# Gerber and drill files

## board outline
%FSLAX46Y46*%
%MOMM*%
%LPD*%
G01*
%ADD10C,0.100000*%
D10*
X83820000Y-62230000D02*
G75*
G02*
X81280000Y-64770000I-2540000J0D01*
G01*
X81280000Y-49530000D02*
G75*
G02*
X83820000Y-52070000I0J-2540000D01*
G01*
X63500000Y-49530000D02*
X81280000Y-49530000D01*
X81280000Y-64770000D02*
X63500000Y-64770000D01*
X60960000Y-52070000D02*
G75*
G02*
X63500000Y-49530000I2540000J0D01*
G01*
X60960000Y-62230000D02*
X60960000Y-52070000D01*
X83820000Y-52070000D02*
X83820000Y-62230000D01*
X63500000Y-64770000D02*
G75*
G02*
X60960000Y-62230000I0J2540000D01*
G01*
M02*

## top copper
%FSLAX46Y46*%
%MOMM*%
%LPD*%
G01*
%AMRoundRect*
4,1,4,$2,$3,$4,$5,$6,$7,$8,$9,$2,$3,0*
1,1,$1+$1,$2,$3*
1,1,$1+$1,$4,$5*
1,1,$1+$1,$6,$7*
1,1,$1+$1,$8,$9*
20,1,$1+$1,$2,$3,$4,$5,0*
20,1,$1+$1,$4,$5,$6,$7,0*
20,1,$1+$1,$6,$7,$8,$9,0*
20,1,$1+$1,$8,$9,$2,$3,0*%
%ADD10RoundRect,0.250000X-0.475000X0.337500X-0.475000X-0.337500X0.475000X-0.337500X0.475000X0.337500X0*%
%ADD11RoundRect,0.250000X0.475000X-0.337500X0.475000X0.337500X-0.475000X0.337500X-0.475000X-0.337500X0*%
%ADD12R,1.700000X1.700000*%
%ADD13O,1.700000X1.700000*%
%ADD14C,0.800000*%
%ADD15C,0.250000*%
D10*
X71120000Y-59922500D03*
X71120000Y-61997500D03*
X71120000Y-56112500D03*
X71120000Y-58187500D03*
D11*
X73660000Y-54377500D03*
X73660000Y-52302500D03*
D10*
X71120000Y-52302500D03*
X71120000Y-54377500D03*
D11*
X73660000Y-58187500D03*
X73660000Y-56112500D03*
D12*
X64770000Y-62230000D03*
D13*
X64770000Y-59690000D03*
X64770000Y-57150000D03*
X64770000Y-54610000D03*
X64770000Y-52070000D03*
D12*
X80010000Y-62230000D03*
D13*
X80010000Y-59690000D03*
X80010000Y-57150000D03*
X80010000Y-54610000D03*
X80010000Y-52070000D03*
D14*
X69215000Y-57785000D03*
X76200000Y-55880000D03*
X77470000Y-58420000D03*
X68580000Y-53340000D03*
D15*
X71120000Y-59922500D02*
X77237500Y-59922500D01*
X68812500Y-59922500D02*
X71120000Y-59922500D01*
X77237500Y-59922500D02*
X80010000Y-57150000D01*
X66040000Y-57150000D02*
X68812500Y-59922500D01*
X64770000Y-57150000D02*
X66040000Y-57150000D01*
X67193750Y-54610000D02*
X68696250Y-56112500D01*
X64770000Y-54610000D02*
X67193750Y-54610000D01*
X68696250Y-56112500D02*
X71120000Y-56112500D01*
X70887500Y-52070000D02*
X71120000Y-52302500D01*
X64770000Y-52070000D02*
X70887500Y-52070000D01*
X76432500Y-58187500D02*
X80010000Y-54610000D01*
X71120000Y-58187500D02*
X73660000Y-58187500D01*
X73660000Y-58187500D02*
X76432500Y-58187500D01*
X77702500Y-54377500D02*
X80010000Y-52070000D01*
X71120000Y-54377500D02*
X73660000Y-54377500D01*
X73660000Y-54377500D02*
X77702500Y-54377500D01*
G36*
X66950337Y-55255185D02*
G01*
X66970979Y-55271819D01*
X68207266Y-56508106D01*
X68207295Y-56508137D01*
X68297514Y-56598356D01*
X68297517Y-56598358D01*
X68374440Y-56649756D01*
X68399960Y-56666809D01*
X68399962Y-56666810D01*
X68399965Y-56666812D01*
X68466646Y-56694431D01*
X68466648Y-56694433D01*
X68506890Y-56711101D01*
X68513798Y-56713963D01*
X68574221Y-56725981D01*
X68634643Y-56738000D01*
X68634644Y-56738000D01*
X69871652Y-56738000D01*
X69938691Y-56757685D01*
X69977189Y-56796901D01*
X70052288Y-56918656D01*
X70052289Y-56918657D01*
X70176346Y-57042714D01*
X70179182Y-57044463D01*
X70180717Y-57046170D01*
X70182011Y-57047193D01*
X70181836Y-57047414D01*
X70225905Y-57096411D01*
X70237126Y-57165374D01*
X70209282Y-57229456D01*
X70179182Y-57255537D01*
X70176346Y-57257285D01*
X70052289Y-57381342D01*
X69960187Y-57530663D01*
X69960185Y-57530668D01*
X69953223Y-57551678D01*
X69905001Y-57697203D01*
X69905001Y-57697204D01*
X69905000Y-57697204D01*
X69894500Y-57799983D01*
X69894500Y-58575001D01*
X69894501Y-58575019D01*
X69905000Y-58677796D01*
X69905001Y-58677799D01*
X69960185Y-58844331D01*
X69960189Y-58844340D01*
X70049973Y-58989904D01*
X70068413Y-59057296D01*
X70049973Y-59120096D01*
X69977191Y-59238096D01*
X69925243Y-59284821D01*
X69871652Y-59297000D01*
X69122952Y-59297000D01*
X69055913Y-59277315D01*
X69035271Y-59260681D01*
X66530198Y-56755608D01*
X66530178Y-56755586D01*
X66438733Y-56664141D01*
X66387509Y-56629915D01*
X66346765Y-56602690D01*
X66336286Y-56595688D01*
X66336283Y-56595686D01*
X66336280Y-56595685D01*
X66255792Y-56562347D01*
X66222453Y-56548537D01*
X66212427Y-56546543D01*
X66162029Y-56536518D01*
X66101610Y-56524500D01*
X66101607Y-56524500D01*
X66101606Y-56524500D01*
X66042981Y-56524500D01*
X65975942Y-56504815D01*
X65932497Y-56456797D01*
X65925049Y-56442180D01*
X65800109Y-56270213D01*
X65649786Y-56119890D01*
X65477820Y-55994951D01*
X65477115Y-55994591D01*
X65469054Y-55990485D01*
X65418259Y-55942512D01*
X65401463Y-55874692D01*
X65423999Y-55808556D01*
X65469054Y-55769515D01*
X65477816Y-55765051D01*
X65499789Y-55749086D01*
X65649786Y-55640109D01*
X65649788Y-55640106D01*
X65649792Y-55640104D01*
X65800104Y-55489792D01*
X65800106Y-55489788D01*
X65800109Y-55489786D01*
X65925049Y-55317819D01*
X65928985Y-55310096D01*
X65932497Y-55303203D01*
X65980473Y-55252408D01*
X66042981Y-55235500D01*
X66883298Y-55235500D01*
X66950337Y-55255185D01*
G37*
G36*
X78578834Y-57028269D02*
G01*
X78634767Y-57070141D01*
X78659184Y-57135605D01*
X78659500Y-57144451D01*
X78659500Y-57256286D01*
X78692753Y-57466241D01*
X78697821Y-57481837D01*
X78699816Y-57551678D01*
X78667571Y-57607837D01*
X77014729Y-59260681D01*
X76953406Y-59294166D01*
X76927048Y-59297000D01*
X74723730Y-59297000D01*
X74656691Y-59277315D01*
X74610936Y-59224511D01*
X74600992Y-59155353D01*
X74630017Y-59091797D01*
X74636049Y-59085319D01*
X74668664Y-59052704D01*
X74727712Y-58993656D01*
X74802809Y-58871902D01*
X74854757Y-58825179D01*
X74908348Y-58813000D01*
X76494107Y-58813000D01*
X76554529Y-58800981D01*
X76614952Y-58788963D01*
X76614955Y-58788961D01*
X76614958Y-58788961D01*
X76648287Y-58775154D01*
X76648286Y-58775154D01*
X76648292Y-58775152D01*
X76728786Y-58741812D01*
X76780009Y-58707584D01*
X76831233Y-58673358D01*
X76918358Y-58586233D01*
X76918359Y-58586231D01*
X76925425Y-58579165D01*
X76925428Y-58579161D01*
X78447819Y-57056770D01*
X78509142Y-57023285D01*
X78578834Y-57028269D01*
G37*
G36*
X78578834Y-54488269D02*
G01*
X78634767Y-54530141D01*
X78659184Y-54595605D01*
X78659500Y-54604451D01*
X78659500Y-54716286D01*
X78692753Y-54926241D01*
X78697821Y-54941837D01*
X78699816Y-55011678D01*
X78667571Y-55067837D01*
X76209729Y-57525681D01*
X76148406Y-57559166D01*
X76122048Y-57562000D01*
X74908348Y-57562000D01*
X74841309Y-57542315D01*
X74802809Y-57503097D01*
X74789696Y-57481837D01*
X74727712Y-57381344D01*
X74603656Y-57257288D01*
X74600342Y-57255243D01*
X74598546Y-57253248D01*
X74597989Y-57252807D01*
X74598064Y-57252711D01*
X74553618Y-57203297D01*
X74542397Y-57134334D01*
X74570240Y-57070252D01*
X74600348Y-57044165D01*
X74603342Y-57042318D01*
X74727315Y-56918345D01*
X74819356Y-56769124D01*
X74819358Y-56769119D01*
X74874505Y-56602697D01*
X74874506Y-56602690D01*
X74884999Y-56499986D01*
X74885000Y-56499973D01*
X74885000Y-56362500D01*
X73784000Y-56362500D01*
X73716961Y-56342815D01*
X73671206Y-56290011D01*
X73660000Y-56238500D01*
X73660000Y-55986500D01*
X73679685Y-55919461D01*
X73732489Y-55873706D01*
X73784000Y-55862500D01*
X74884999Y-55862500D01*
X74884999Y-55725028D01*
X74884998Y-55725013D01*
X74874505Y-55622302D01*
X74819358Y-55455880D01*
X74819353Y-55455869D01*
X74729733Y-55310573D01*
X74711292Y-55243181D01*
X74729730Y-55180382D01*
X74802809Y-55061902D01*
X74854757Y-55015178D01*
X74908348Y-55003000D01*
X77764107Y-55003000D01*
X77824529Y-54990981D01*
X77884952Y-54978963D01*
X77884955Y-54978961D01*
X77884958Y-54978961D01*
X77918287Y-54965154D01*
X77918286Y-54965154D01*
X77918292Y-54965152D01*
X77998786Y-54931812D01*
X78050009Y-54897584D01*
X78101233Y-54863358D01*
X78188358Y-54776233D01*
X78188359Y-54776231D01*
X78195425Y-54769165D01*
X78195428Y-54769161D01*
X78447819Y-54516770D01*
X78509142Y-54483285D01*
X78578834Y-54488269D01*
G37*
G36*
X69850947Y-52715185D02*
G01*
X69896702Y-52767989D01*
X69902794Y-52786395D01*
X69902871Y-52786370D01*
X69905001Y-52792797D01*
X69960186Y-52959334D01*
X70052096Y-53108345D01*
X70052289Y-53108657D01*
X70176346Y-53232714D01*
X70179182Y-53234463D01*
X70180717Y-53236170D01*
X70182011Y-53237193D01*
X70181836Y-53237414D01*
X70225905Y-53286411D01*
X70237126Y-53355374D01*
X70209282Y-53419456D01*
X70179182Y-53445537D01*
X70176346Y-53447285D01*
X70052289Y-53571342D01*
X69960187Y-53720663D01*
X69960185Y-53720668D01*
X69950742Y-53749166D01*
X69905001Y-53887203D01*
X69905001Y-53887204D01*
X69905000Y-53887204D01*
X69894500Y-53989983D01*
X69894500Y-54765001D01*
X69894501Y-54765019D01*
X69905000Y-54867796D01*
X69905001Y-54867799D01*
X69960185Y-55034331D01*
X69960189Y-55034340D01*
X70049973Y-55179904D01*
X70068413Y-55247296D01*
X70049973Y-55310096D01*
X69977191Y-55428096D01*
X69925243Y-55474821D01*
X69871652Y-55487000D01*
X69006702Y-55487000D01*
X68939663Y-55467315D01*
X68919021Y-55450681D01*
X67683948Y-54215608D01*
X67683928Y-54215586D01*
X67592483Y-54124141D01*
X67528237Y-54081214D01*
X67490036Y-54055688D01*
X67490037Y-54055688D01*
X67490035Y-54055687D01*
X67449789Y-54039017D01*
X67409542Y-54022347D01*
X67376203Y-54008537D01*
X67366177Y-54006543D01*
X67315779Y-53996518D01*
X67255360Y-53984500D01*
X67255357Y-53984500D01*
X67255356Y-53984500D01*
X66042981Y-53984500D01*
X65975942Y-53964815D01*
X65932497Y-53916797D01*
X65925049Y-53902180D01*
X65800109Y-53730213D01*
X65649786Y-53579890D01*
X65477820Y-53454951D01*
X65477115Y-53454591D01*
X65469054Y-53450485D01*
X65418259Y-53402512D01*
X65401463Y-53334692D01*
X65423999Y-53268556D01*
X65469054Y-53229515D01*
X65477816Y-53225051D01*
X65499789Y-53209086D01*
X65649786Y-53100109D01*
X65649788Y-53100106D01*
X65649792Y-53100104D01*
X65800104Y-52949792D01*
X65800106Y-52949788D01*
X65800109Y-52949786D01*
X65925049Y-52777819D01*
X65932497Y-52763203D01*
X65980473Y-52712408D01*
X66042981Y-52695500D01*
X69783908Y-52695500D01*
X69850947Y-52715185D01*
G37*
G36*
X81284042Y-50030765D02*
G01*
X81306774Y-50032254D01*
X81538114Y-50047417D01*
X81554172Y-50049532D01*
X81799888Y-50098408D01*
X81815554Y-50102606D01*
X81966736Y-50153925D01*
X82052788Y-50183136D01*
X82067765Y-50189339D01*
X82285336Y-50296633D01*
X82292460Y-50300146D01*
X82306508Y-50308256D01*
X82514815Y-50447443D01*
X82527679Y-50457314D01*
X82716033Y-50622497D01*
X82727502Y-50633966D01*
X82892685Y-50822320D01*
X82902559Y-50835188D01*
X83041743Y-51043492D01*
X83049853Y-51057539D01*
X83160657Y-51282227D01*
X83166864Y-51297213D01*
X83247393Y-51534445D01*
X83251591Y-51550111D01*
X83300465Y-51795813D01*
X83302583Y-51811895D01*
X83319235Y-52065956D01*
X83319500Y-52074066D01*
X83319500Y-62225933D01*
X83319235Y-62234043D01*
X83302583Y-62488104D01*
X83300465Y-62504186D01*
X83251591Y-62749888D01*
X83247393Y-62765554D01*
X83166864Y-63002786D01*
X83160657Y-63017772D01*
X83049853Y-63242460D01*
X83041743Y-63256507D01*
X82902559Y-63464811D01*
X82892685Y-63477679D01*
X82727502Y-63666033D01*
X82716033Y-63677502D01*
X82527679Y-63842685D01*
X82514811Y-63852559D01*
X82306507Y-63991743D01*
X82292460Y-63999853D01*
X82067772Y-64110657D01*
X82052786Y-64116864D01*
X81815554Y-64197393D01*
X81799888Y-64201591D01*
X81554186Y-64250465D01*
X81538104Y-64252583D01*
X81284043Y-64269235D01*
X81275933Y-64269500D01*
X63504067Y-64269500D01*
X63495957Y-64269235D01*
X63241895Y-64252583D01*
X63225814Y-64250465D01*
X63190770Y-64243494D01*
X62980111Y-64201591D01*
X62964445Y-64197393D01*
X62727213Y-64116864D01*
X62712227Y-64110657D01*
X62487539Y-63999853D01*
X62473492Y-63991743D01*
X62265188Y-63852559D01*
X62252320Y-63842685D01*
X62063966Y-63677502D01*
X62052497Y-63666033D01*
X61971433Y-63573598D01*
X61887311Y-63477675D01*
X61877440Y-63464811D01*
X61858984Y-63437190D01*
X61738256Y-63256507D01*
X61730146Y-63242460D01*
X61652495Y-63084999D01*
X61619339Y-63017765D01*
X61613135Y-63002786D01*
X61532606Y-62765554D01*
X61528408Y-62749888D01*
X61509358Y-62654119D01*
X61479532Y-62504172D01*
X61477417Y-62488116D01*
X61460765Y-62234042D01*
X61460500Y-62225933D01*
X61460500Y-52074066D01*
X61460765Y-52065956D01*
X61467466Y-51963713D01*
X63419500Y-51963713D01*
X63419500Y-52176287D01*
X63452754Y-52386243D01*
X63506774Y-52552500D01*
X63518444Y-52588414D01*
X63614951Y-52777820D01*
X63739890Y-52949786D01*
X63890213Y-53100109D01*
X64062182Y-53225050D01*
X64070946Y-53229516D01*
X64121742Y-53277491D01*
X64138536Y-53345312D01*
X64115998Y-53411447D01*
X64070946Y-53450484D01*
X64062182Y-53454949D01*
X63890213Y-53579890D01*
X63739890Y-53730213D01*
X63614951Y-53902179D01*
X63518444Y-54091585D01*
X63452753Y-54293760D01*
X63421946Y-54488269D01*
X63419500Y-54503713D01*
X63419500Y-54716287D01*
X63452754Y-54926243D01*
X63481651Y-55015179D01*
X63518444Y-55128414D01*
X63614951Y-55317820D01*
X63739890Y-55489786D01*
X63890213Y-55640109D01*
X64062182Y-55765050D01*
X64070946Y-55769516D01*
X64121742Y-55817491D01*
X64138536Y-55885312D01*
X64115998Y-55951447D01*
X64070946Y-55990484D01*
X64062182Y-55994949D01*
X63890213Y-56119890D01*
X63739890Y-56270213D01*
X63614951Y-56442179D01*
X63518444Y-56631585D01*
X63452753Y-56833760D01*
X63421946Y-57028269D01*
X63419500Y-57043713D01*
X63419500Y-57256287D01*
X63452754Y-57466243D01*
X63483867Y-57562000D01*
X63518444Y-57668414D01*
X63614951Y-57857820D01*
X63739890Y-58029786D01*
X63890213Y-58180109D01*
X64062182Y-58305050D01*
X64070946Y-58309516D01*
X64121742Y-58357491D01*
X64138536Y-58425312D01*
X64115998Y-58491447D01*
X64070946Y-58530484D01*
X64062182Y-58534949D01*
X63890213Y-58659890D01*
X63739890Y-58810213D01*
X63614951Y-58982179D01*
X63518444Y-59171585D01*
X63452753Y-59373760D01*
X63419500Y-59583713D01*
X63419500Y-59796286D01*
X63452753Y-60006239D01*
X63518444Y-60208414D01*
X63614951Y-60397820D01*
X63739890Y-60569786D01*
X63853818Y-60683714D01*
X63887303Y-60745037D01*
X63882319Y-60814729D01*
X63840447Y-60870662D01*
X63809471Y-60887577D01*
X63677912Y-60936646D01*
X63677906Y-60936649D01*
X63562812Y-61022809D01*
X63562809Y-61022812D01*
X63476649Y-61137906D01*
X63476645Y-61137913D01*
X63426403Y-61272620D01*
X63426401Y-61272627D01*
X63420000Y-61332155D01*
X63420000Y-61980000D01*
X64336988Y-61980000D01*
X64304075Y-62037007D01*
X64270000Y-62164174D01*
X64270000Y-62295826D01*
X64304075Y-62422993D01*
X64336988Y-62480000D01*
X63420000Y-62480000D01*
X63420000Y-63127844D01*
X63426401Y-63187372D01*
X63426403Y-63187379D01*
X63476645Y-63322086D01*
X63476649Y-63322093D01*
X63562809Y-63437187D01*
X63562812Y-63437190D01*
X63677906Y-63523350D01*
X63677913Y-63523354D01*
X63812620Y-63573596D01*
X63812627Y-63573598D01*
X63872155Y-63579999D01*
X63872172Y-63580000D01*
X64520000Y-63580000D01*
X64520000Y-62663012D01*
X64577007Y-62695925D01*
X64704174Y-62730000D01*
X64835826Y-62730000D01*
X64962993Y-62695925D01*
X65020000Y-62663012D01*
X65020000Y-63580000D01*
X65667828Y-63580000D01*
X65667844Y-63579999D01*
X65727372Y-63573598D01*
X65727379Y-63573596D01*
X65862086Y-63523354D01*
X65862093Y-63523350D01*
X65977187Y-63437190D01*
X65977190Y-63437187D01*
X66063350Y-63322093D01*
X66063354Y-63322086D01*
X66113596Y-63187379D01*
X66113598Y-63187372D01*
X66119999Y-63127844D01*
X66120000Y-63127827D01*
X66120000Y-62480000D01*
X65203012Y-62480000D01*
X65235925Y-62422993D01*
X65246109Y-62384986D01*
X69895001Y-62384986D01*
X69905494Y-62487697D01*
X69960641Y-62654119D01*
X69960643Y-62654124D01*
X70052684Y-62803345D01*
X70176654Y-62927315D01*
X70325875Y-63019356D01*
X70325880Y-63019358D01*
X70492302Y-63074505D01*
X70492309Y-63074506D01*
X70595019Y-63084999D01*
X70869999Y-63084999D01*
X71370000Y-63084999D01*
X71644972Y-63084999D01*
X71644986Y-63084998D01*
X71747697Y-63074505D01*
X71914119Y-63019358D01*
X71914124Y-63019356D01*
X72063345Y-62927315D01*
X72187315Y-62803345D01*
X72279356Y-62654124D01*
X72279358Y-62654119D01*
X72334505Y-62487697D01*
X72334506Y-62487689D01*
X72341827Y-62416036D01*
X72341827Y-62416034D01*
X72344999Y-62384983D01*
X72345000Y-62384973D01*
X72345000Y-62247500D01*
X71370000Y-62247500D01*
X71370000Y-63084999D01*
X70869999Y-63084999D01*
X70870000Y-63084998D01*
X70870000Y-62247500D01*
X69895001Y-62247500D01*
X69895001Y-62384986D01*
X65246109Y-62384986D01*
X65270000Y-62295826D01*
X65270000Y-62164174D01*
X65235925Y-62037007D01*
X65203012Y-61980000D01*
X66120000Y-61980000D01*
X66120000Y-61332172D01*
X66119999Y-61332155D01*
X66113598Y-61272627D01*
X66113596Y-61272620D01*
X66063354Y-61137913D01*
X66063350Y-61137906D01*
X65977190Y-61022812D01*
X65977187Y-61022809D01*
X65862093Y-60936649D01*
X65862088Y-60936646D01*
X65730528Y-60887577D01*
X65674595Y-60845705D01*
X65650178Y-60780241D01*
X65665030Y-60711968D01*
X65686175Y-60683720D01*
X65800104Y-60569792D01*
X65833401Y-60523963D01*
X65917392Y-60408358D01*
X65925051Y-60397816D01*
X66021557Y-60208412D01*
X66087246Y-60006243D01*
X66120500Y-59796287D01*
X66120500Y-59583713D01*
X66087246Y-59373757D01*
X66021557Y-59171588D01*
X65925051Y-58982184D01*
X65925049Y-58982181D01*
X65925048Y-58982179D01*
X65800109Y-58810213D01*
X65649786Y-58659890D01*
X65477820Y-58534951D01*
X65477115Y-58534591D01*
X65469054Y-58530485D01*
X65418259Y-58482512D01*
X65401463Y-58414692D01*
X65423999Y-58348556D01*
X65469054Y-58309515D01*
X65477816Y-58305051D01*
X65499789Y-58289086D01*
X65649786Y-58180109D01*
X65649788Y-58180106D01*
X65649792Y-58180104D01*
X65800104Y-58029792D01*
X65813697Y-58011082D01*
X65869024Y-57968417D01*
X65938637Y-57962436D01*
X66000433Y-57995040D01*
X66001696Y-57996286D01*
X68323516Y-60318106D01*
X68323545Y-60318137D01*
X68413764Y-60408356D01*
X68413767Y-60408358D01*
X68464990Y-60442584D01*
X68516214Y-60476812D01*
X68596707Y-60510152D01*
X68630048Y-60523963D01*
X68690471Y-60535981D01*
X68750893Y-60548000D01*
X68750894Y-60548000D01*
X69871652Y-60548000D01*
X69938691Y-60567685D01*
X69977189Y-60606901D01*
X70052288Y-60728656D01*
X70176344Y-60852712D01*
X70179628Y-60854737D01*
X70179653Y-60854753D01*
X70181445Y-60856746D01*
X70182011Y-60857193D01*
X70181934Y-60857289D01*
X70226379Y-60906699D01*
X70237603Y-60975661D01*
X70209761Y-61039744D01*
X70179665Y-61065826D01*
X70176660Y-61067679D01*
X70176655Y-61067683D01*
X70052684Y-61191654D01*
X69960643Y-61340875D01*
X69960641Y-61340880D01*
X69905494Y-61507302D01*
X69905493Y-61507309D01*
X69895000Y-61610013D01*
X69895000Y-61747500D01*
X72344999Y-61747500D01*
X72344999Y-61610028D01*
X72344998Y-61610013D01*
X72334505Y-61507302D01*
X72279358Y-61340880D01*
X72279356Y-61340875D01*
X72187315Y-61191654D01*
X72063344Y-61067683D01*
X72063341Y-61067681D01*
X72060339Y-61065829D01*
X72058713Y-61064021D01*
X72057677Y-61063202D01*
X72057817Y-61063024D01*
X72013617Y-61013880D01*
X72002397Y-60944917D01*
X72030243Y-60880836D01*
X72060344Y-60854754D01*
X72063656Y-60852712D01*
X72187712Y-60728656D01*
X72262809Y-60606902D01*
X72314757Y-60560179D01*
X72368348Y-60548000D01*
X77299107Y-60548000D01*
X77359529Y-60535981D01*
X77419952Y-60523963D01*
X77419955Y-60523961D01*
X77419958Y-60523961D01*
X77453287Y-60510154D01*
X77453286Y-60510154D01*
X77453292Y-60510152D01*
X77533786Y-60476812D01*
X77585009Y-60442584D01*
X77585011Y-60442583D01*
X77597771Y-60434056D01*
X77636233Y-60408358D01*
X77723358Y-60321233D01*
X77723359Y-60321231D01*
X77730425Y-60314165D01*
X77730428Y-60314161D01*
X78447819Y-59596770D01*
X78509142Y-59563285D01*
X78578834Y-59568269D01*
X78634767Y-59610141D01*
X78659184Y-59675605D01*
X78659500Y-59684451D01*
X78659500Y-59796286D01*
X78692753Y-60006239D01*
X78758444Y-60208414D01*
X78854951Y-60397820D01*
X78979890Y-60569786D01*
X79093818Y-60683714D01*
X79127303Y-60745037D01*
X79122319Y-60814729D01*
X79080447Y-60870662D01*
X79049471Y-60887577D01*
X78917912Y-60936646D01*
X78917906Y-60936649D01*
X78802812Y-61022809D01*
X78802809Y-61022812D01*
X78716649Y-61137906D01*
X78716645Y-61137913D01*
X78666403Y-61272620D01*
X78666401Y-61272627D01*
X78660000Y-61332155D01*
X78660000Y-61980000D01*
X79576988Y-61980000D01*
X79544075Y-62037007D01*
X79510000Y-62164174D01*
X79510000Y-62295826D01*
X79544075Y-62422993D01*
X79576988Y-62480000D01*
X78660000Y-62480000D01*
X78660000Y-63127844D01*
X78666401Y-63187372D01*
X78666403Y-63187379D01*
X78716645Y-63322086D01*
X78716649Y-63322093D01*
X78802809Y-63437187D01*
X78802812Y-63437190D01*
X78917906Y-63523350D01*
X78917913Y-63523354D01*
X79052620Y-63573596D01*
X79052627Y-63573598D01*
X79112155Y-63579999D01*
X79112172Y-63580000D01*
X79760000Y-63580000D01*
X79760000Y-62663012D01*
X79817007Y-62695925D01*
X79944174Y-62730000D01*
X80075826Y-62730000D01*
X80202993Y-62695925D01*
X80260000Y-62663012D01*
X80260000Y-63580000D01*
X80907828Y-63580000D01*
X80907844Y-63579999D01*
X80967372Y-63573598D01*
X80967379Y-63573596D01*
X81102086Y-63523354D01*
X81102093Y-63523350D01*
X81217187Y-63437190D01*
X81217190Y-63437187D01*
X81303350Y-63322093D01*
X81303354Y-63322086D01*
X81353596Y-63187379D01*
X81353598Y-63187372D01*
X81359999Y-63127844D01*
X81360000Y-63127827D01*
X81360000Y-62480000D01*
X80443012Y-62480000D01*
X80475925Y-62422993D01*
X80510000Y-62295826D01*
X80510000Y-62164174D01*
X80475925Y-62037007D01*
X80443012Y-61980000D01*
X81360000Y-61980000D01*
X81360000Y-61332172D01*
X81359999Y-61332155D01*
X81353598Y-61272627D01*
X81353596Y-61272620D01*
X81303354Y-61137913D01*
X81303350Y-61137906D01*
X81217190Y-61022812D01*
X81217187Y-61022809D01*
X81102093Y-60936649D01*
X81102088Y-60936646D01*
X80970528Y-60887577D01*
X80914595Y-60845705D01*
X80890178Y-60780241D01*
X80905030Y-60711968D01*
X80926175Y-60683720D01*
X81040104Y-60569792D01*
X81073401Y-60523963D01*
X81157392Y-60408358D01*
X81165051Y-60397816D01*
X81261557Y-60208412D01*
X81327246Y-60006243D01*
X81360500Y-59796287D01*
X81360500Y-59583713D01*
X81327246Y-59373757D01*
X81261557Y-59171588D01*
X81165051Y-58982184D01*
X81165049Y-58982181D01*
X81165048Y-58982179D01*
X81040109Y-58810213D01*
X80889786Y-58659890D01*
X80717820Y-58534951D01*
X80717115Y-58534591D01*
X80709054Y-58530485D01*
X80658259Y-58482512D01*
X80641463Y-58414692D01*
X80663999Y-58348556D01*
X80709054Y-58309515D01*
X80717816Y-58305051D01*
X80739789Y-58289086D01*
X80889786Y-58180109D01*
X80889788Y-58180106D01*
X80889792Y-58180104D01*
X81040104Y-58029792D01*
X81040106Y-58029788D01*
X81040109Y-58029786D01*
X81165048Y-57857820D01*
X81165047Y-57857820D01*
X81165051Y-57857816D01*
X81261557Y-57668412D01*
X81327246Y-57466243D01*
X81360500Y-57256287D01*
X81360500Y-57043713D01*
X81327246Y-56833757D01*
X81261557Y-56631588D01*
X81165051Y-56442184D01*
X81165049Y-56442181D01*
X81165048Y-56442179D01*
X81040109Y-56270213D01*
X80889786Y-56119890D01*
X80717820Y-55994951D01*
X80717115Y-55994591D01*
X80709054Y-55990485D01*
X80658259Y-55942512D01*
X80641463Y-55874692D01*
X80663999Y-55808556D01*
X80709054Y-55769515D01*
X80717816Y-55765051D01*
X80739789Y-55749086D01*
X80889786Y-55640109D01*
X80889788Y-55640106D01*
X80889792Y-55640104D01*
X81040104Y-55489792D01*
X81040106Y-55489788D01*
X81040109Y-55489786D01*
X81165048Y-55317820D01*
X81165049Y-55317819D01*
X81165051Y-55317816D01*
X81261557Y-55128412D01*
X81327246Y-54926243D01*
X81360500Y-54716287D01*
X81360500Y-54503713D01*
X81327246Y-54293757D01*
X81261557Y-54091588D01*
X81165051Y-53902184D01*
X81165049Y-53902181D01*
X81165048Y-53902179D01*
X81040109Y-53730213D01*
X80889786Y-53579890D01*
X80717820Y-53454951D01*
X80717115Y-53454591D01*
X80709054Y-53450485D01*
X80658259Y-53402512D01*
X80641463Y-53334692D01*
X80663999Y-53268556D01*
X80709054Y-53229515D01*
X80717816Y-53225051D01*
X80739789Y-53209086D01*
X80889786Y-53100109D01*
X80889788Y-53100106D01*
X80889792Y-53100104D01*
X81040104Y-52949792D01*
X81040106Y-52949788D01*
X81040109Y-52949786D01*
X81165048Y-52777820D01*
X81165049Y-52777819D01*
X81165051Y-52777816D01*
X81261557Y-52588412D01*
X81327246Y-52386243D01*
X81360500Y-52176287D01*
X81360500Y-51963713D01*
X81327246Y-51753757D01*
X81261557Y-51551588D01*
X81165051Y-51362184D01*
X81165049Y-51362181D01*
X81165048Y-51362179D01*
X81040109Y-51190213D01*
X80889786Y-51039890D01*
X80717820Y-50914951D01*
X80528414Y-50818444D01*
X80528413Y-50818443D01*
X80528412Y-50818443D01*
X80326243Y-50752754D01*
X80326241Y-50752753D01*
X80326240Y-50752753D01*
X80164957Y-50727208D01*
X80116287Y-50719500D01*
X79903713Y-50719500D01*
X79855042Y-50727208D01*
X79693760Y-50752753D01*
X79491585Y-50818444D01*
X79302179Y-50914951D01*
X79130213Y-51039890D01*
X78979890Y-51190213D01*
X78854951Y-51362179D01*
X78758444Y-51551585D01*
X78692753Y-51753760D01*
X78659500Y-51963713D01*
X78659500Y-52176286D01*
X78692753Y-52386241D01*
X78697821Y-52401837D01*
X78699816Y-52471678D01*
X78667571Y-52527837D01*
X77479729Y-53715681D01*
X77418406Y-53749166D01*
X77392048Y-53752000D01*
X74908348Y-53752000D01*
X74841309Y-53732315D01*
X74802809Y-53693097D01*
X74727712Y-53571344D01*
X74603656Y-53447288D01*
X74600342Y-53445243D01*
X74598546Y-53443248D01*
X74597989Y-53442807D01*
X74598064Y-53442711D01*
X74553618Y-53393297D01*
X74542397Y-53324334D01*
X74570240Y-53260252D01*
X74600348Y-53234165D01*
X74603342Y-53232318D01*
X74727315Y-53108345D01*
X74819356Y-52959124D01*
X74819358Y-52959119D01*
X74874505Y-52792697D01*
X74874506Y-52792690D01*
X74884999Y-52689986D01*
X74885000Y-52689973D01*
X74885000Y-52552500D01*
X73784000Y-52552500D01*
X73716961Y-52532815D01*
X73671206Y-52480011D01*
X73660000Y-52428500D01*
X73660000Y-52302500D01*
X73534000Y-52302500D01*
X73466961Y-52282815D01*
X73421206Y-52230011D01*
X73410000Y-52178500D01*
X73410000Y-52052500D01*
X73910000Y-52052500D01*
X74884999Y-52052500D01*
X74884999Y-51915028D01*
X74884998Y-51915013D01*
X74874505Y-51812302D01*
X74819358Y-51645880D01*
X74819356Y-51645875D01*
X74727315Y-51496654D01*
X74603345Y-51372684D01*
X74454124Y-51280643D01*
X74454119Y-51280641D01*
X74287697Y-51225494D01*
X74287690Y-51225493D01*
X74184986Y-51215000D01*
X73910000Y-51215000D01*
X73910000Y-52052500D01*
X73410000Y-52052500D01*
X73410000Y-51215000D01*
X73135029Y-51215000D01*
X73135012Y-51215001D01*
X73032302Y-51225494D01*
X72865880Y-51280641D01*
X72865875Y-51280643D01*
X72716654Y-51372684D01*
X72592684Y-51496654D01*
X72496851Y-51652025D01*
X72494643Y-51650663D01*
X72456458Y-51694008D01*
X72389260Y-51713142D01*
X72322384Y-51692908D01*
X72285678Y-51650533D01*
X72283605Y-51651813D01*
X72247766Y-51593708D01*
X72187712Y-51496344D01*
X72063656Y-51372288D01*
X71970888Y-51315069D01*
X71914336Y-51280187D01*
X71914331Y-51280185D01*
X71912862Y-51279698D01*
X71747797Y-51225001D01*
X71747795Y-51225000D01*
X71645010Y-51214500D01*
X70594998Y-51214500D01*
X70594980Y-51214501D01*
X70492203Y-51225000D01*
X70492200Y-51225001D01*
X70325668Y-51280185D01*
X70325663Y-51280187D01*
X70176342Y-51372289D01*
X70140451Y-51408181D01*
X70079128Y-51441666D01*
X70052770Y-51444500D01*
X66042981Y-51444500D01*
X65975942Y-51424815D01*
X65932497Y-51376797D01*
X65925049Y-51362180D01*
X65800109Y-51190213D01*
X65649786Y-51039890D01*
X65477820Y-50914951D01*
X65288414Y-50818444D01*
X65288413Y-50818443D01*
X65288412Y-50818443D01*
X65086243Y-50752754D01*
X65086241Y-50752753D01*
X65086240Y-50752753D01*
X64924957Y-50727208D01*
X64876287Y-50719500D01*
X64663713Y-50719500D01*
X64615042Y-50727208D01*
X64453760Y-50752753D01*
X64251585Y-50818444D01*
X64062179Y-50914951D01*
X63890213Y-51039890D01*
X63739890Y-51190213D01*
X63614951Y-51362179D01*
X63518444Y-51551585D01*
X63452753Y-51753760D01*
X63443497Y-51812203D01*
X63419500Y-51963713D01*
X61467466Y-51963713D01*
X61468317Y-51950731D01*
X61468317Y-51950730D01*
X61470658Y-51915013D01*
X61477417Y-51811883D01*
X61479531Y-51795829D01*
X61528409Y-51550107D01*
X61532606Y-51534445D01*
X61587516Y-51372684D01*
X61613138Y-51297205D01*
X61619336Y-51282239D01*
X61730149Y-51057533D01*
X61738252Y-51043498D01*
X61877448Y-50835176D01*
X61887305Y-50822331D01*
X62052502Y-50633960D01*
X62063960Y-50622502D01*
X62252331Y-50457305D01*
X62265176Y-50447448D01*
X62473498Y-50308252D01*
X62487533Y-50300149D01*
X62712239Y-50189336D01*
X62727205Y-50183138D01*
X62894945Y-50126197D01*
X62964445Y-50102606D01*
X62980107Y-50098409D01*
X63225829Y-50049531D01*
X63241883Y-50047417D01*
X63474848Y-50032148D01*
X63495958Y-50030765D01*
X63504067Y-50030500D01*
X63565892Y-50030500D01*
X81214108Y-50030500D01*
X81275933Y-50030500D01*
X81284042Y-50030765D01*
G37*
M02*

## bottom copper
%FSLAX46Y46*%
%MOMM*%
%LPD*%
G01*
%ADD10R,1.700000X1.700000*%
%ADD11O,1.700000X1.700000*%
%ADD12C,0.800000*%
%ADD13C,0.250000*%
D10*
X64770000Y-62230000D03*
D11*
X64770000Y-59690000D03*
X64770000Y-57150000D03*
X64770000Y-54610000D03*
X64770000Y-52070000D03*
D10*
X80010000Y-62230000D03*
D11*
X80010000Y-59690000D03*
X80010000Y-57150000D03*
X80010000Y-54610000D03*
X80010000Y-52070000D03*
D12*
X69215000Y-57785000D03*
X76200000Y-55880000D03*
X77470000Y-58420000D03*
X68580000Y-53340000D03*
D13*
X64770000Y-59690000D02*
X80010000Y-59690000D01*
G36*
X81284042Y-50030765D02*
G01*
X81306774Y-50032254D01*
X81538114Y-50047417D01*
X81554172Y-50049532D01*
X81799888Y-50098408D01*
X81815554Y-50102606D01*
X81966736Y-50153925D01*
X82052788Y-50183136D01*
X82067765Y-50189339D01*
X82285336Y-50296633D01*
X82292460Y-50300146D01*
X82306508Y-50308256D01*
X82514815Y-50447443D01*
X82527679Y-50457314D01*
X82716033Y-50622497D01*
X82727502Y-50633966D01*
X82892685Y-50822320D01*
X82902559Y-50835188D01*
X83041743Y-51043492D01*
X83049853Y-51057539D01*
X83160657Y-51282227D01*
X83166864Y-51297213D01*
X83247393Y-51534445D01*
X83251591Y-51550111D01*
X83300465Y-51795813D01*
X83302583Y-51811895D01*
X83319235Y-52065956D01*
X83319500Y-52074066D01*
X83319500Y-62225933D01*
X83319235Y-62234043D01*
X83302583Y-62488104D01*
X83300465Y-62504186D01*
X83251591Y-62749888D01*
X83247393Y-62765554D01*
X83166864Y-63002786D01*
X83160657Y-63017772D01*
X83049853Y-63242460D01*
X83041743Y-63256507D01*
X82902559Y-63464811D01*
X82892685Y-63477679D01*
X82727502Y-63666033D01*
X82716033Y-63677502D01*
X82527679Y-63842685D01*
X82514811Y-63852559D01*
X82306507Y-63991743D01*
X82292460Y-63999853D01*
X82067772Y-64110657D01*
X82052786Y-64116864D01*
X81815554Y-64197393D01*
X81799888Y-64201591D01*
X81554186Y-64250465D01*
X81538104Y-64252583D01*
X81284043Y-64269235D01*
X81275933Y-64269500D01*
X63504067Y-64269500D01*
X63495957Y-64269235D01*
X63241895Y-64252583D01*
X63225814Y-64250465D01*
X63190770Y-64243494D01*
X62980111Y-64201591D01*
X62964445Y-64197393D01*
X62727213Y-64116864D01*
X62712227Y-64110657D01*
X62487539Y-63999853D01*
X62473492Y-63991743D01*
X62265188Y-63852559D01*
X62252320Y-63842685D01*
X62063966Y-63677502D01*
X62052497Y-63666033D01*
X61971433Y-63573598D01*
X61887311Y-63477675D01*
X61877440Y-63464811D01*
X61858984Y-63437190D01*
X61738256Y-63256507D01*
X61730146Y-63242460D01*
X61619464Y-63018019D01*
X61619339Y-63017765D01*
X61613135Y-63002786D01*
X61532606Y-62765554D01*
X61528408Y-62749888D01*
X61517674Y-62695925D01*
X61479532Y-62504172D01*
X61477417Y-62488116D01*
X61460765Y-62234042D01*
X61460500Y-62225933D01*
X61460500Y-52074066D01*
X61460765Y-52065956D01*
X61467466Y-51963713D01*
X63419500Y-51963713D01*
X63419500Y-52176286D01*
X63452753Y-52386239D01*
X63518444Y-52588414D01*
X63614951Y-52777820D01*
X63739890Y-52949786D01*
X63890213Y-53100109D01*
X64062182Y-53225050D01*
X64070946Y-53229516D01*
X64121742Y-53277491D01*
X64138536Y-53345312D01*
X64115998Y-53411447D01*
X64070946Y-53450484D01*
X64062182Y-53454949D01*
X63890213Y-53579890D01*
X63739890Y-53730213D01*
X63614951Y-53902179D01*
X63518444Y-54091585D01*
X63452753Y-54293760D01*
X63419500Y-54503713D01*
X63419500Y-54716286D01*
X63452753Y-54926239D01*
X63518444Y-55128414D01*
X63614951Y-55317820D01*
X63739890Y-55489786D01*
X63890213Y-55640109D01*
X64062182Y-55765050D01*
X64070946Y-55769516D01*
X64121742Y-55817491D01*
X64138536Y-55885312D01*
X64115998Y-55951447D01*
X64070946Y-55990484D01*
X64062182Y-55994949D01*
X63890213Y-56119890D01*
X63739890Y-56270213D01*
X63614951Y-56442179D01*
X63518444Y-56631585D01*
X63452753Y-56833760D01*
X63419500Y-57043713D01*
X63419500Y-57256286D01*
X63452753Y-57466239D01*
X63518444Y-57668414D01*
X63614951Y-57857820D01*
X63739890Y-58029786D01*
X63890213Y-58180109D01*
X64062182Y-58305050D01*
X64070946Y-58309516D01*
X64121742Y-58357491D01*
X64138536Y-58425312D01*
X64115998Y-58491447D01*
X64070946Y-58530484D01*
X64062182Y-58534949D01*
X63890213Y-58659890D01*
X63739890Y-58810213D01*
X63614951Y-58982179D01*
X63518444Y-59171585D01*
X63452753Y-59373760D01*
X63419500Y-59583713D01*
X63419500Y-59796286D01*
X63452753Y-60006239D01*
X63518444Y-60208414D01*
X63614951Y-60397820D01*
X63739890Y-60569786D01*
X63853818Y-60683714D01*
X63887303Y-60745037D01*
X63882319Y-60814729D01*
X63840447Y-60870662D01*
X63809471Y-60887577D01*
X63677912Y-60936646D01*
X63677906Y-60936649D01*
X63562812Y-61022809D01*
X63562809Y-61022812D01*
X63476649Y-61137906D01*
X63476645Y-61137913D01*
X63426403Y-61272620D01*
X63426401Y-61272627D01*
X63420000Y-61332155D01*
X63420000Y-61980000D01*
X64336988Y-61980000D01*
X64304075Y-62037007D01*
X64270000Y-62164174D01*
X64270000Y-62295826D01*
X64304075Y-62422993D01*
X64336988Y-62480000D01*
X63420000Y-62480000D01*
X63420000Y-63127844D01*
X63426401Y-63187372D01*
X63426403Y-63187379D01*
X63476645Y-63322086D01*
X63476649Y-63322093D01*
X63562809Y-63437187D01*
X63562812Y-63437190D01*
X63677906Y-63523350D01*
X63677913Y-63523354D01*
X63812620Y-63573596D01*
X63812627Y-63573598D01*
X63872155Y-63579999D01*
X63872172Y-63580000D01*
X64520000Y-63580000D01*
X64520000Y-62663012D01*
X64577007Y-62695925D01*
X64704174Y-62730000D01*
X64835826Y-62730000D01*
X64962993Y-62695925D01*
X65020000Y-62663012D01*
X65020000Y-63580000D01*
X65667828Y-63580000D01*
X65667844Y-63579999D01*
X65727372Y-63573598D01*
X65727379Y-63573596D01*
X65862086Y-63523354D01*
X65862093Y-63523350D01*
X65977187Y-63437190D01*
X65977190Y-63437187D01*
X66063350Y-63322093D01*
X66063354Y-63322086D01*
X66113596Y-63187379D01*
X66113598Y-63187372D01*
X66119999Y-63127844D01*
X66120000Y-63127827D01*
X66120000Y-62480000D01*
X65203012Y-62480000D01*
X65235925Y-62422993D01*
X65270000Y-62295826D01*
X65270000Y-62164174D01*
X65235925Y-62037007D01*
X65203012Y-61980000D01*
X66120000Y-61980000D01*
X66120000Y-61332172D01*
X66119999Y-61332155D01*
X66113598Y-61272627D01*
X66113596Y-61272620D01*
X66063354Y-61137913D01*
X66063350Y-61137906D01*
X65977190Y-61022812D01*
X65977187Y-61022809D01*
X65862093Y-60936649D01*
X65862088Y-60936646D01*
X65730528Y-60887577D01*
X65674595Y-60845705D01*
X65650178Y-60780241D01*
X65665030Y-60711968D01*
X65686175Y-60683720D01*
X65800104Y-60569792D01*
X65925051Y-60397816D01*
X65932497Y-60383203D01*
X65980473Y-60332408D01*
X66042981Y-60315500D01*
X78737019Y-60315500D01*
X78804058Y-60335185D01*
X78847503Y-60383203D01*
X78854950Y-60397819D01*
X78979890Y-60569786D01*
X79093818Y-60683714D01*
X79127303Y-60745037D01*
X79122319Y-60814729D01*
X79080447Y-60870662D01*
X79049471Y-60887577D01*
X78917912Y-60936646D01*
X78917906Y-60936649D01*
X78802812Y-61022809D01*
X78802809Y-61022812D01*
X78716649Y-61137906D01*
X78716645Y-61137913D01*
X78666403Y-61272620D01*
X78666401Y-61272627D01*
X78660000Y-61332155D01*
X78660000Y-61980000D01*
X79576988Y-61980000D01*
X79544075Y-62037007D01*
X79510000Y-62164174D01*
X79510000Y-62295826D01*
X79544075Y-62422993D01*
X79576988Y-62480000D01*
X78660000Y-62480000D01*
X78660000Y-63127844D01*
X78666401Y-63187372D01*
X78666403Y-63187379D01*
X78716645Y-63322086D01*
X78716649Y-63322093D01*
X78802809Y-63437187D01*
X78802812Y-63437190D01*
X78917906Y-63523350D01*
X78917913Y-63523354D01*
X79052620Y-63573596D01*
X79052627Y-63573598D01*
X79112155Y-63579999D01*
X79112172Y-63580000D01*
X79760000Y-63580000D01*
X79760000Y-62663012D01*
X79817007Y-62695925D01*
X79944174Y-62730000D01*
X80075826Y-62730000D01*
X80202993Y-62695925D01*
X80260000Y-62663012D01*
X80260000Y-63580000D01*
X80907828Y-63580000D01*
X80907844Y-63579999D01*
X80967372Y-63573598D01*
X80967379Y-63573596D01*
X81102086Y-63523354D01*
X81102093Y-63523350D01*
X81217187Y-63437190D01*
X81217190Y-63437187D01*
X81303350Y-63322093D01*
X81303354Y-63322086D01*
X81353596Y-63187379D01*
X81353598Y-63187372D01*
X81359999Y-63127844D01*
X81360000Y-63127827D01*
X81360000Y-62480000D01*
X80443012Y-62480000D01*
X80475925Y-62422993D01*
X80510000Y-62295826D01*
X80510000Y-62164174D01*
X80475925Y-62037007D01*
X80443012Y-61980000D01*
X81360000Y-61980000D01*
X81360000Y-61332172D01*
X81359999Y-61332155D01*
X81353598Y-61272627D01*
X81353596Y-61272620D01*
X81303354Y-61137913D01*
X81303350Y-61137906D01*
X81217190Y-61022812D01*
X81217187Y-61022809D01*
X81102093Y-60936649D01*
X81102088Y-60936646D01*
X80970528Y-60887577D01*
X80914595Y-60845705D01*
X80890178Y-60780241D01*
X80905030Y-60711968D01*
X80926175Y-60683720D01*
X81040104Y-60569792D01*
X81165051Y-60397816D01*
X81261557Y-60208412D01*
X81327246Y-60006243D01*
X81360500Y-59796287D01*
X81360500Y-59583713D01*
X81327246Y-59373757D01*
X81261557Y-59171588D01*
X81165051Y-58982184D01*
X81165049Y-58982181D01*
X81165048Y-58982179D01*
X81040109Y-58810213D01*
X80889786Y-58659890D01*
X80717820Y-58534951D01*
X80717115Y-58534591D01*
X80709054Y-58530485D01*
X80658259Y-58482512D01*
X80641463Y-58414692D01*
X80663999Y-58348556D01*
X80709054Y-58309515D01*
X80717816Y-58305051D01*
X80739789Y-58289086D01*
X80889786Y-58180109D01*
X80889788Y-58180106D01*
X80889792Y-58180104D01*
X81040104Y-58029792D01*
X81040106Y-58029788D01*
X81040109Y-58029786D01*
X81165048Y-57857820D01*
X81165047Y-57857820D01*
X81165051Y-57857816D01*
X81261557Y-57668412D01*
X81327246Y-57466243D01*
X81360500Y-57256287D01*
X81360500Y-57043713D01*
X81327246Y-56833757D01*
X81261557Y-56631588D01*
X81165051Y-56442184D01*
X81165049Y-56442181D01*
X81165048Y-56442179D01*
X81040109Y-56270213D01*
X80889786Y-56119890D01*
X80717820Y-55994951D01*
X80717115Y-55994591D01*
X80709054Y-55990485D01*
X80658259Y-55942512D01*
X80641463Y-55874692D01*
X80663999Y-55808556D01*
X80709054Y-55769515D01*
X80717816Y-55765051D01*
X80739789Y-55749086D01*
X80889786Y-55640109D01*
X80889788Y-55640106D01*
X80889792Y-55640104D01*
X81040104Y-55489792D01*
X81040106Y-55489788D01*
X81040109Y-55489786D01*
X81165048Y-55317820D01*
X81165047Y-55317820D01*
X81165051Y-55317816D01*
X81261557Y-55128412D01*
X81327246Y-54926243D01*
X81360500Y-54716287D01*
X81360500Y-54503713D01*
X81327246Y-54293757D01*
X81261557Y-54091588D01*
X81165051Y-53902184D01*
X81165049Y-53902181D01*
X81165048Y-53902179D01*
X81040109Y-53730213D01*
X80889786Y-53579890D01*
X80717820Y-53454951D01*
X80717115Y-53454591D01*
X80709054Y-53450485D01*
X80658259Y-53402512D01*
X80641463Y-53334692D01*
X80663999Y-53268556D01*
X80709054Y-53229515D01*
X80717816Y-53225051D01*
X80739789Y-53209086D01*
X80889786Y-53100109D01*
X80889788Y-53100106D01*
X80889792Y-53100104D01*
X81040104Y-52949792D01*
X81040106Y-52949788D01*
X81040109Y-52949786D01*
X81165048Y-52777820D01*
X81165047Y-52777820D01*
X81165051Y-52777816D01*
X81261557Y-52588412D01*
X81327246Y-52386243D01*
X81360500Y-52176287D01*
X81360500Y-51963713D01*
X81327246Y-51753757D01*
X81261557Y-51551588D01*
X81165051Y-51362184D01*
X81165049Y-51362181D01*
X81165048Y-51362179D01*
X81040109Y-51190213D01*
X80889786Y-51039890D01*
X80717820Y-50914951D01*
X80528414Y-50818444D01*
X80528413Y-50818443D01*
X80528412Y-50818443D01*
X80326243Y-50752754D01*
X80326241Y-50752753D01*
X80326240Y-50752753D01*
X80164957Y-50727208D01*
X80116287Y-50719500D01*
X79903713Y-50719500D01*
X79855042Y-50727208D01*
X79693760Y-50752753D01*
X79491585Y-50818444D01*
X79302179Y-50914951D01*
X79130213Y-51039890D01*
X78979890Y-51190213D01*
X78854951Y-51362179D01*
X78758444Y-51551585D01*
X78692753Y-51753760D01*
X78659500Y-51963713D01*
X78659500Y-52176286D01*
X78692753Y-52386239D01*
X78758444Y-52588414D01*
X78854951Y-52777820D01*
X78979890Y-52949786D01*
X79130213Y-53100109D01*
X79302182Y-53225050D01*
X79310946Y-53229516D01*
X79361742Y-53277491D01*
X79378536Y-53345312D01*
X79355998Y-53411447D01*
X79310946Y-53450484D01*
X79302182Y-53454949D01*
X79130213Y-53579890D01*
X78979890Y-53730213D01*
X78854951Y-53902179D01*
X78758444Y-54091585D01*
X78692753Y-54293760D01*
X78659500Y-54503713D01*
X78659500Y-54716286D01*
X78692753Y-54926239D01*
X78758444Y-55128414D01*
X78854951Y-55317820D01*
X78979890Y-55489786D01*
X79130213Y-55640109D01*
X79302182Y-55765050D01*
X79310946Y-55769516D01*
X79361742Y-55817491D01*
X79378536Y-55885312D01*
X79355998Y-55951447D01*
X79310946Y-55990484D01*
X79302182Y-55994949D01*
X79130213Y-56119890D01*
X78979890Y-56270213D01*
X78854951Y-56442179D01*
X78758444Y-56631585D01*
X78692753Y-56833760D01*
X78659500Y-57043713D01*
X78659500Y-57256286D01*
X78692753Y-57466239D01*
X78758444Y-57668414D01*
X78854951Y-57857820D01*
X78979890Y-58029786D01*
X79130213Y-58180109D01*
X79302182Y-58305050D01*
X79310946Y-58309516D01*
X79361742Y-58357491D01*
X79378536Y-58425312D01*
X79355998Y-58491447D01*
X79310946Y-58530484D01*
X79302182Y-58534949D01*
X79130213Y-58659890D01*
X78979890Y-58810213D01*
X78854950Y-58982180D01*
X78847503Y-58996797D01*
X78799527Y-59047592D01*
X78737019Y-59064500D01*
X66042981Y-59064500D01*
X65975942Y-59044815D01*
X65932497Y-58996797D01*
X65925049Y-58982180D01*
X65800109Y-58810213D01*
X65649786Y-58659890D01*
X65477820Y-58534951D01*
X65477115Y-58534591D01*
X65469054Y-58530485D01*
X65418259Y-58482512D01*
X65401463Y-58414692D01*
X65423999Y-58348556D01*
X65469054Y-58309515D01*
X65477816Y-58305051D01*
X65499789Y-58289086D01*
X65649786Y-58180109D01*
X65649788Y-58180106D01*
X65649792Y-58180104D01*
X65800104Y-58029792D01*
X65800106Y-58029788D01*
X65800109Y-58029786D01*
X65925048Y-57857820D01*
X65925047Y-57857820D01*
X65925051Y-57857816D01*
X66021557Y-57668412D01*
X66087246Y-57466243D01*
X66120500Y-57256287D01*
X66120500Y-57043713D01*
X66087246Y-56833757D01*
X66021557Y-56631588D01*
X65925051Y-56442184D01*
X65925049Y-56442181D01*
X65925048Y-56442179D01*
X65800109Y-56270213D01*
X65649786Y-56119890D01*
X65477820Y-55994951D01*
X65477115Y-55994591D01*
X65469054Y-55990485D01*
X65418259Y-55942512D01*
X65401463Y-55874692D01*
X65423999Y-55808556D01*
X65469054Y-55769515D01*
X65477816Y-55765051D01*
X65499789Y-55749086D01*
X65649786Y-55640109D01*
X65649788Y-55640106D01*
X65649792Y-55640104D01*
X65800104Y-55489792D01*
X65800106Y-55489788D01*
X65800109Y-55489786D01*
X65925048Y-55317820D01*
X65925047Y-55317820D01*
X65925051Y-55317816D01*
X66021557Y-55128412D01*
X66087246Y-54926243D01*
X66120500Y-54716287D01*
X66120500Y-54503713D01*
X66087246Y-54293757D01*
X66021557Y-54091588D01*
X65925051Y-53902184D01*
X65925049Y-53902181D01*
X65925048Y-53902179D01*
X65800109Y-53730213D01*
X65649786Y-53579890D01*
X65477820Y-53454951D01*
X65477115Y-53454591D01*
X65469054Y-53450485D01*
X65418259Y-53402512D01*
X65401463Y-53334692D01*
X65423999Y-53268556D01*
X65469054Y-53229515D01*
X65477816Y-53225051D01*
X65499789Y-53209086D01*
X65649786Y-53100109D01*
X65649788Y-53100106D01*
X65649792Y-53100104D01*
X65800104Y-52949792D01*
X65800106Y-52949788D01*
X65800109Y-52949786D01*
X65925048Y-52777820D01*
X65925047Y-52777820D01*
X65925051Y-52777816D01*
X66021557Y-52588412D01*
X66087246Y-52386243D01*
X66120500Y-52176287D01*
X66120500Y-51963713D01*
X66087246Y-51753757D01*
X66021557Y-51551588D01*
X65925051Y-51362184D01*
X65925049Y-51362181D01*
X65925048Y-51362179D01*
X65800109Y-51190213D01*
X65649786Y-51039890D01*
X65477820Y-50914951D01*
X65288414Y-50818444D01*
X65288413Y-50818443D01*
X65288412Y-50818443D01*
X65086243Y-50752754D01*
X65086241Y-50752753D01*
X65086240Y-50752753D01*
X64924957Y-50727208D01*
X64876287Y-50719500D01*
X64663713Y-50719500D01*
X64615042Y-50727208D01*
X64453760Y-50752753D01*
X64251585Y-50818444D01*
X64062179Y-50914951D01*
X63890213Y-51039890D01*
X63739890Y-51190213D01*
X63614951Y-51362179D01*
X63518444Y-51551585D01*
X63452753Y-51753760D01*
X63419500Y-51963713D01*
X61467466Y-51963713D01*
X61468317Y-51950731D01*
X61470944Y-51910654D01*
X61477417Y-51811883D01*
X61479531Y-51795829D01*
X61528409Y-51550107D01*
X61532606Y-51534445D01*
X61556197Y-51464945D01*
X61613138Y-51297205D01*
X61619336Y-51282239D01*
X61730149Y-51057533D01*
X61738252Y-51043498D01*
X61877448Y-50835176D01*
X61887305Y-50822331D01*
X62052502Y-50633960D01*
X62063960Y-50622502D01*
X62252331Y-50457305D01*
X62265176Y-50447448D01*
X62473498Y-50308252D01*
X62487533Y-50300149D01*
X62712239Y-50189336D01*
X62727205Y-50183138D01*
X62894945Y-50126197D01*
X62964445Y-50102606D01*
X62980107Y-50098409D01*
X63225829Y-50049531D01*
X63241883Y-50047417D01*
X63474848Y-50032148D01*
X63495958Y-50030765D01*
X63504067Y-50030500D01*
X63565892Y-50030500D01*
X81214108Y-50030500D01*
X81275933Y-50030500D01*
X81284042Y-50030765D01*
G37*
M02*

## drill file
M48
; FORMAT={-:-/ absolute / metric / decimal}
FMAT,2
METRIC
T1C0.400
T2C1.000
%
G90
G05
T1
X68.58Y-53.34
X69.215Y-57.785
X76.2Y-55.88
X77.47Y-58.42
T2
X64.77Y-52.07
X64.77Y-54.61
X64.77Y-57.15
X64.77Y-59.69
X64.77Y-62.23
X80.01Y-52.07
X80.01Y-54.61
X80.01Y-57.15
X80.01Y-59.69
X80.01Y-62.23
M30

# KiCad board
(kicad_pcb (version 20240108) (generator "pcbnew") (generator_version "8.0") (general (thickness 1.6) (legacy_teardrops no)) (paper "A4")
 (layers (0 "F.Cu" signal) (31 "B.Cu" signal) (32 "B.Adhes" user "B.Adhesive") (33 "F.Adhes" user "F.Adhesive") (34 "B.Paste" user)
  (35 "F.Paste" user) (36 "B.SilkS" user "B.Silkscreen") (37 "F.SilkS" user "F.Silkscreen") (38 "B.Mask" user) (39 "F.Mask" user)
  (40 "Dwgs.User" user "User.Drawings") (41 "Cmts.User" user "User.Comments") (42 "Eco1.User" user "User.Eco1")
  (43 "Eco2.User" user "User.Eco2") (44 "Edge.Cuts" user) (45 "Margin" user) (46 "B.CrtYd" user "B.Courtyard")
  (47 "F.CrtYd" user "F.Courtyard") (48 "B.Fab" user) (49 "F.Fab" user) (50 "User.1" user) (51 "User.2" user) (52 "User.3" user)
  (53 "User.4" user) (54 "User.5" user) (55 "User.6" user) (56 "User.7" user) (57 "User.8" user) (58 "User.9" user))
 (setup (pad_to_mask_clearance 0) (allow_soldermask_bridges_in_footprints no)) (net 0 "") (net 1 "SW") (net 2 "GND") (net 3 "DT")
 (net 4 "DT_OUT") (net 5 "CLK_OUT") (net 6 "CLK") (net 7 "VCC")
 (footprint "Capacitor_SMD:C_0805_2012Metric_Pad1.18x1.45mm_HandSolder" (layer "F.Cu") (at 71.12 60.96 -90)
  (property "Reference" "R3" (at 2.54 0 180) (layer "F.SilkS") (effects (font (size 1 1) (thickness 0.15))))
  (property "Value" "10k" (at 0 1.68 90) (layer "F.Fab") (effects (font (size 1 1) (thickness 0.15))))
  (pad "1" smd roundrect (at -1.0375 0 270) (size 1.175 1.45) (layers "F.Cu" "F.Paste" "F.Mask") (roundrect_rratio 0.2127659574)
   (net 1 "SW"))
  (pad "2" smd roundrect (at 1.0375 0 270) (size 1.175 1.45) (layers "F.Cu" "F.Paste" "F.Mask") (roundrect_rratio 0.2127659574)
   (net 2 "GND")))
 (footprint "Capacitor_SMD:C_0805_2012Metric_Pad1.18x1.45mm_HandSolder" (layer "F.Cu") (at 71.12 57.15 -90)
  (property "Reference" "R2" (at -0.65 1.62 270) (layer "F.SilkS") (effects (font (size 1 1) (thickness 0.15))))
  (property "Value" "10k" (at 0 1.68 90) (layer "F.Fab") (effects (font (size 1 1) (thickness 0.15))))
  (pad "1" smd roundrect (at -1.0375 0 270) (size 1.175 1.45) (layers "F.Cu" "F.Paste" "F.Mask") (roundrect_rratio 0.2127659574)
   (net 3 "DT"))
  (pad "2" smd roundrect (at 1.0375 0 270) (size 1.175 1.45) (layers "F.Cu" "F.Paste" "F.Mask") (roundrect_rratio 0.2127659574)
   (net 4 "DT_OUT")))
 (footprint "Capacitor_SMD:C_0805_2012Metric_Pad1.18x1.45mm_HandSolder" (layer "F.Cu") (at 73.66 53.34 90)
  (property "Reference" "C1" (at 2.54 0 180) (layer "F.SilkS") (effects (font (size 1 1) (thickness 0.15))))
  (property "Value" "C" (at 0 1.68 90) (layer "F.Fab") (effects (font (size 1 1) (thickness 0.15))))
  (pad "1" smd roundrect (at -1.0375 0 90) (size 1.175 1.45) (layers "F.Cu" "F.Paste" "F.Mask") (roundrect_rratio 0.2127659574)
   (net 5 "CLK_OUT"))
  (pad "2" smd roundrect (at 1.0375 0 90) (size 1.175 1.45) (layers "F.Cu" "F.Paste" "F.Mask") (roundrect_rratio 0.2127659574) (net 2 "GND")))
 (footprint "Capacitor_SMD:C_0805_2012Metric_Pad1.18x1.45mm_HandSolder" (layer "F.Cu") (at 71.12 53.34 -90)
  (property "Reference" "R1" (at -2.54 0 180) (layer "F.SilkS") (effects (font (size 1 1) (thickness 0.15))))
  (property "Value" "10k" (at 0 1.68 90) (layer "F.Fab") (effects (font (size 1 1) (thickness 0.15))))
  (pad "1" smd roundrect (at -1.0375 0 270) (size 1.175 1.45) (layers "F.Cu" "F.Paste" "F.Mask") (roundrect_rratio 0.2127659574)
   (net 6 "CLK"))
  (pad "2" smd roundrect (at 1.0375 0 270) (size 1.175 1.45) (layers "F.Cu" "F.Paste" "F.Mask") (roundrect_rratio 0.2127659574)
   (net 5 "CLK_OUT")))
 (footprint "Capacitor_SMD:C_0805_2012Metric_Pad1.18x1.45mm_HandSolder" (layer "F.Cu") (at 73.66 57.15 90)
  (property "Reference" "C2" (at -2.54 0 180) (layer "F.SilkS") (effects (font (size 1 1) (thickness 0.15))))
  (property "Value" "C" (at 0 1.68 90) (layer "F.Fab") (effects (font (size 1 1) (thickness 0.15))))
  (pad "1" smd roundrect (at -1.0375 0 90) (size 1.175 1.45) (layers "F.Cu" "F.Paste" "F.Mask") (roundrect_rratio 0.2127659574)
   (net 4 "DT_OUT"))
  (pad "2" smd roundrect (at 1.0375 0 90) (size 1.175 1.45) (layers "F.Cu" "F.Paste" "F.Mask") (roundrect_rratio 0.2127659574) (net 2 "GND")))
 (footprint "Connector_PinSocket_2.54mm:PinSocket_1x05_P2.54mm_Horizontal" (layer "B.Cu") (at 64.77 62.23)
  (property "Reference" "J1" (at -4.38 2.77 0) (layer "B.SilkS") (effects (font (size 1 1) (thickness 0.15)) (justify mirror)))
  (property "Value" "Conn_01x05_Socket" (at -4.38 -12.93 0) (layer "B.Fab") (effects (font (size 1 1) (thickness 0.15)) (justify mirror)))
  (pad "1" thru_hole rect (at 0 0) (size 1.7 1.7) (drill 1) (layers "*.Cu" "*.Mask") (remove_unused_layers no) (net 2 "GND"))
  (pad "2" thru_hole oval (at 0 -2.54) (size 1.7 1.7) (drill 1) (layers "*.Cu" "*.Mask") (remove_unused_layers no) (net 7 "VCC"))
  (pad "3" thru_hole oval (at 0 -5.08) (size 1.7 1.7) (drill 1) (layers "*.Cu" "*.Mask") (remove_unused_layers no) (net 1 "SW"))
  (pad "4" thru_hole oval (at 0 -7.62) (size 1.7 1.7) (drill 1) (layers "*.Cu" "*.Mask") (remove_unused_layers no) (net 3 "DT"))
  (pad "5" thru_hole oval (at 0 -10.16) (size 1.7 1.7) (drill 1) (layers "*.Cu" "*.Mask") (remove_unused_layers no) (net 6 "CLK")))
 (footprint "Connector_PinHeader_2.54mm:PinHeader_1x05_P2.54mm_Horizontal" (layer "B.Cu") (at 80.01 62.23)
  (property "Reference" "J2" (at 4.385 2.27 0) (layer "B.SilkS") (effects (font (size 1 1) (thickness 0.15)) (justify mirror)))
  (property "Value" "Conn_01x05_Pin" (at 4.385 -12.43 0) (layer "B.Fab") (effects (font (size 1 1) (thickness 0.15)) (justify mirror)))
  (pad "1" thru_hole rect (at 0 0) (size 1.7 1.7) (drill 1) (layers "*.Cu" "*.Mask") (remove_unused_layers no) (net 2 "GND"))
  (pad "2" thru_hole oval (at 0 -2.54) (size 1.7 1.7) (drill 1) (layers "*.Cu" "*.Mask") (remove_unused_layers no) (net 7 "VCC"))
  (pad "3" thru_hole oval (at 0 -5.08) (size 1.7 1.7) (drill 1) (layers "*.Cu" "*.Mask") (remove_unused_layers no) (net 1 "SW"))
  (pad "4" thru_hole oval (at 0 -7.62) (size 1.7 1.7) (drill 1) (layers "*.Cu" "*.Mask") (remove_unused_layers no) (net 4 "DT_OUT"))
  (pad "5" thru_hole oval (at 0 -10.16) (size 1.7 1.7) (drill 1) (layers "*.Cu" "*.Mask") (remove_unused_layers no) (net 5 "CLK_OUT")))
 (gr_arc (start 83.82 62.23) (mid 83.076051 64.026051) (end 81.28 64.77) (stroke (width 0.1) (type default)) (layer "Edge.Cuts"))
 (gr_arc (start 81.28 49.53) (mid 83.076051 50.273949) (end 83.82 52.07) (stroke (width 0.1) (type default)) (layer "Edge.Cuts"))
 (gr_line (start 63.5 49.53) (end 81.28 49.53) (stroke (width 0.1) (type default)) (layer "Edge.Cuts"))
 (gr_line (start 81.28 64.77) (end 63.5 64.77) (stroke (width 0.1) (type default)) (layer "Edge.Cuts"))
 (gr_arc (start 60.96 52.07) (mid 61.703949 50.273949) (end 63.5 49.53) (stroke (width 0.1) (type default)) (layer "Edge.Cuts"))
 (gr_line (start 60.96 62.23) (end 60.96 52.07) (stroke (width 0.1) (type default)) (layer "Edge.Cuts"))
 (gr_line (start 83.82 52.07) (end 83.82 62.23) (stroke (width 0.1) (type default)) (layer "Edge.Cuts"))
 (gr_arc (start 63.5 64.77) (mid 61.703949 64.026051) (end 60.96 62.23) (stroke (width 0.1) (type default)) (layer "Edge.Cuts"))
 (via (at 69.215 57.785) (size 0.8) (drill 0.4) (layers "F.Cu" "B.Cu") (free yes) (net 2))
 (via (at 76.2 55.88) (size 0.8) (drill 0.4) (layers "F.Cu" "B.Cu") (free yes) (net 2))
 (via (at 77.47 58.42) (size 0.8) (drill 0.4) (layers "F.Cu" "B.Cu") (free yes) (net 2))
 (via (at 68.58 53.34) (size 0.8) (drill 0.4) (layers "F.Cu" "B.Cu") (free yes) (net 2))
 (segment (start 64.77 59.69) (end 80.01 59.69) (width 0.25) (layer "B.Cu") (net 7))
 (segment (start 71.12 59.9225) (end 77.2375 59.9225) (width 0.25) (layer "F.Cu") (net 1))
 (segment (start 68.8125 59.9225) (end 71.12 59.9225) (width 0.25) (layer "F.Cu") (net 1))
 (segment (start 77.2375 59.9225) (end 80.01 57.15) (width 0.25) (layer "F.Cu") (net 1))
 (segment (start 66.04 57.15) (end 68.8125 59.9225) (width 0.25) (layer "F.Cu") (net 1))
 (segment (start 64.77 57.15) (end 66.04 57.15) (width 0.25) (layer "F.Cu") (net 1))
 (segment (start 67.19375 54.61) (end 68.69625 56.1125) (width 0.25) (layer "F.Cu") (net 3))
 (segment (start 64.77 54.61) (end 67.19375 54.61) (width 0.25) (layer "F.Cu") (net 3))
 (segment (start 68.69625 56.1125) (end 71.12 56.1125) (width 0.25) (layer "F.Cu") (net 3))
 (segment (start 70.8875 52.07) (end 71.12 52.3025) (width 0.25) (layer "F.Cu") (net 6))
 (segment (start 64.77 52.07) (end 70.8875 52.07) (width 0.25) (layer "F.Cu") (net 6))
 (segment (start 76.4325 58.1875) (end 80.01 54.61) (width 0.25) (layer "F.Cu") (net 4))
 (segment (start 71.12 58.1875) (end 73.66 58.1875) (width 0.25) (layer "F.Cu") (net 4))
 (segment (start 73.66 58.1875) (end 76.4325 58.1875) (width 0.25) (layer "F.Cu") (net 4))
 (segment (start 77.7025 54.3775) (end 80.01 52.07) (width 0.25) (layer "F.Cu") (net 5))
 (segment (start 71.12 54.3775) (end 73.66 54.3775) (width 0.25) (layer "F.Cu") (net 5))
 (segment (start 73.66 54.3775) (end 77.7025 54.3775) (width 0.25) (layer "F.Cu") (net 5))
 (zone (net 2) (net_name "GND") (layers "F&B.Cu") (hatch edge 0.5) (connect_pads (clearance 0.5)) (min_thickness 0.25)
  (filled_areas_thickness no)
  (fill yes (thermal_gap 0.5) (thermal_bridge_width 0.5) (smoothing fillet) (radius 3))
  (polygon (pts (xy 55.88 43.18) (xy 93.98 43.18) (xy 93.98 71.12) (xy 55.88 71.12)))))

